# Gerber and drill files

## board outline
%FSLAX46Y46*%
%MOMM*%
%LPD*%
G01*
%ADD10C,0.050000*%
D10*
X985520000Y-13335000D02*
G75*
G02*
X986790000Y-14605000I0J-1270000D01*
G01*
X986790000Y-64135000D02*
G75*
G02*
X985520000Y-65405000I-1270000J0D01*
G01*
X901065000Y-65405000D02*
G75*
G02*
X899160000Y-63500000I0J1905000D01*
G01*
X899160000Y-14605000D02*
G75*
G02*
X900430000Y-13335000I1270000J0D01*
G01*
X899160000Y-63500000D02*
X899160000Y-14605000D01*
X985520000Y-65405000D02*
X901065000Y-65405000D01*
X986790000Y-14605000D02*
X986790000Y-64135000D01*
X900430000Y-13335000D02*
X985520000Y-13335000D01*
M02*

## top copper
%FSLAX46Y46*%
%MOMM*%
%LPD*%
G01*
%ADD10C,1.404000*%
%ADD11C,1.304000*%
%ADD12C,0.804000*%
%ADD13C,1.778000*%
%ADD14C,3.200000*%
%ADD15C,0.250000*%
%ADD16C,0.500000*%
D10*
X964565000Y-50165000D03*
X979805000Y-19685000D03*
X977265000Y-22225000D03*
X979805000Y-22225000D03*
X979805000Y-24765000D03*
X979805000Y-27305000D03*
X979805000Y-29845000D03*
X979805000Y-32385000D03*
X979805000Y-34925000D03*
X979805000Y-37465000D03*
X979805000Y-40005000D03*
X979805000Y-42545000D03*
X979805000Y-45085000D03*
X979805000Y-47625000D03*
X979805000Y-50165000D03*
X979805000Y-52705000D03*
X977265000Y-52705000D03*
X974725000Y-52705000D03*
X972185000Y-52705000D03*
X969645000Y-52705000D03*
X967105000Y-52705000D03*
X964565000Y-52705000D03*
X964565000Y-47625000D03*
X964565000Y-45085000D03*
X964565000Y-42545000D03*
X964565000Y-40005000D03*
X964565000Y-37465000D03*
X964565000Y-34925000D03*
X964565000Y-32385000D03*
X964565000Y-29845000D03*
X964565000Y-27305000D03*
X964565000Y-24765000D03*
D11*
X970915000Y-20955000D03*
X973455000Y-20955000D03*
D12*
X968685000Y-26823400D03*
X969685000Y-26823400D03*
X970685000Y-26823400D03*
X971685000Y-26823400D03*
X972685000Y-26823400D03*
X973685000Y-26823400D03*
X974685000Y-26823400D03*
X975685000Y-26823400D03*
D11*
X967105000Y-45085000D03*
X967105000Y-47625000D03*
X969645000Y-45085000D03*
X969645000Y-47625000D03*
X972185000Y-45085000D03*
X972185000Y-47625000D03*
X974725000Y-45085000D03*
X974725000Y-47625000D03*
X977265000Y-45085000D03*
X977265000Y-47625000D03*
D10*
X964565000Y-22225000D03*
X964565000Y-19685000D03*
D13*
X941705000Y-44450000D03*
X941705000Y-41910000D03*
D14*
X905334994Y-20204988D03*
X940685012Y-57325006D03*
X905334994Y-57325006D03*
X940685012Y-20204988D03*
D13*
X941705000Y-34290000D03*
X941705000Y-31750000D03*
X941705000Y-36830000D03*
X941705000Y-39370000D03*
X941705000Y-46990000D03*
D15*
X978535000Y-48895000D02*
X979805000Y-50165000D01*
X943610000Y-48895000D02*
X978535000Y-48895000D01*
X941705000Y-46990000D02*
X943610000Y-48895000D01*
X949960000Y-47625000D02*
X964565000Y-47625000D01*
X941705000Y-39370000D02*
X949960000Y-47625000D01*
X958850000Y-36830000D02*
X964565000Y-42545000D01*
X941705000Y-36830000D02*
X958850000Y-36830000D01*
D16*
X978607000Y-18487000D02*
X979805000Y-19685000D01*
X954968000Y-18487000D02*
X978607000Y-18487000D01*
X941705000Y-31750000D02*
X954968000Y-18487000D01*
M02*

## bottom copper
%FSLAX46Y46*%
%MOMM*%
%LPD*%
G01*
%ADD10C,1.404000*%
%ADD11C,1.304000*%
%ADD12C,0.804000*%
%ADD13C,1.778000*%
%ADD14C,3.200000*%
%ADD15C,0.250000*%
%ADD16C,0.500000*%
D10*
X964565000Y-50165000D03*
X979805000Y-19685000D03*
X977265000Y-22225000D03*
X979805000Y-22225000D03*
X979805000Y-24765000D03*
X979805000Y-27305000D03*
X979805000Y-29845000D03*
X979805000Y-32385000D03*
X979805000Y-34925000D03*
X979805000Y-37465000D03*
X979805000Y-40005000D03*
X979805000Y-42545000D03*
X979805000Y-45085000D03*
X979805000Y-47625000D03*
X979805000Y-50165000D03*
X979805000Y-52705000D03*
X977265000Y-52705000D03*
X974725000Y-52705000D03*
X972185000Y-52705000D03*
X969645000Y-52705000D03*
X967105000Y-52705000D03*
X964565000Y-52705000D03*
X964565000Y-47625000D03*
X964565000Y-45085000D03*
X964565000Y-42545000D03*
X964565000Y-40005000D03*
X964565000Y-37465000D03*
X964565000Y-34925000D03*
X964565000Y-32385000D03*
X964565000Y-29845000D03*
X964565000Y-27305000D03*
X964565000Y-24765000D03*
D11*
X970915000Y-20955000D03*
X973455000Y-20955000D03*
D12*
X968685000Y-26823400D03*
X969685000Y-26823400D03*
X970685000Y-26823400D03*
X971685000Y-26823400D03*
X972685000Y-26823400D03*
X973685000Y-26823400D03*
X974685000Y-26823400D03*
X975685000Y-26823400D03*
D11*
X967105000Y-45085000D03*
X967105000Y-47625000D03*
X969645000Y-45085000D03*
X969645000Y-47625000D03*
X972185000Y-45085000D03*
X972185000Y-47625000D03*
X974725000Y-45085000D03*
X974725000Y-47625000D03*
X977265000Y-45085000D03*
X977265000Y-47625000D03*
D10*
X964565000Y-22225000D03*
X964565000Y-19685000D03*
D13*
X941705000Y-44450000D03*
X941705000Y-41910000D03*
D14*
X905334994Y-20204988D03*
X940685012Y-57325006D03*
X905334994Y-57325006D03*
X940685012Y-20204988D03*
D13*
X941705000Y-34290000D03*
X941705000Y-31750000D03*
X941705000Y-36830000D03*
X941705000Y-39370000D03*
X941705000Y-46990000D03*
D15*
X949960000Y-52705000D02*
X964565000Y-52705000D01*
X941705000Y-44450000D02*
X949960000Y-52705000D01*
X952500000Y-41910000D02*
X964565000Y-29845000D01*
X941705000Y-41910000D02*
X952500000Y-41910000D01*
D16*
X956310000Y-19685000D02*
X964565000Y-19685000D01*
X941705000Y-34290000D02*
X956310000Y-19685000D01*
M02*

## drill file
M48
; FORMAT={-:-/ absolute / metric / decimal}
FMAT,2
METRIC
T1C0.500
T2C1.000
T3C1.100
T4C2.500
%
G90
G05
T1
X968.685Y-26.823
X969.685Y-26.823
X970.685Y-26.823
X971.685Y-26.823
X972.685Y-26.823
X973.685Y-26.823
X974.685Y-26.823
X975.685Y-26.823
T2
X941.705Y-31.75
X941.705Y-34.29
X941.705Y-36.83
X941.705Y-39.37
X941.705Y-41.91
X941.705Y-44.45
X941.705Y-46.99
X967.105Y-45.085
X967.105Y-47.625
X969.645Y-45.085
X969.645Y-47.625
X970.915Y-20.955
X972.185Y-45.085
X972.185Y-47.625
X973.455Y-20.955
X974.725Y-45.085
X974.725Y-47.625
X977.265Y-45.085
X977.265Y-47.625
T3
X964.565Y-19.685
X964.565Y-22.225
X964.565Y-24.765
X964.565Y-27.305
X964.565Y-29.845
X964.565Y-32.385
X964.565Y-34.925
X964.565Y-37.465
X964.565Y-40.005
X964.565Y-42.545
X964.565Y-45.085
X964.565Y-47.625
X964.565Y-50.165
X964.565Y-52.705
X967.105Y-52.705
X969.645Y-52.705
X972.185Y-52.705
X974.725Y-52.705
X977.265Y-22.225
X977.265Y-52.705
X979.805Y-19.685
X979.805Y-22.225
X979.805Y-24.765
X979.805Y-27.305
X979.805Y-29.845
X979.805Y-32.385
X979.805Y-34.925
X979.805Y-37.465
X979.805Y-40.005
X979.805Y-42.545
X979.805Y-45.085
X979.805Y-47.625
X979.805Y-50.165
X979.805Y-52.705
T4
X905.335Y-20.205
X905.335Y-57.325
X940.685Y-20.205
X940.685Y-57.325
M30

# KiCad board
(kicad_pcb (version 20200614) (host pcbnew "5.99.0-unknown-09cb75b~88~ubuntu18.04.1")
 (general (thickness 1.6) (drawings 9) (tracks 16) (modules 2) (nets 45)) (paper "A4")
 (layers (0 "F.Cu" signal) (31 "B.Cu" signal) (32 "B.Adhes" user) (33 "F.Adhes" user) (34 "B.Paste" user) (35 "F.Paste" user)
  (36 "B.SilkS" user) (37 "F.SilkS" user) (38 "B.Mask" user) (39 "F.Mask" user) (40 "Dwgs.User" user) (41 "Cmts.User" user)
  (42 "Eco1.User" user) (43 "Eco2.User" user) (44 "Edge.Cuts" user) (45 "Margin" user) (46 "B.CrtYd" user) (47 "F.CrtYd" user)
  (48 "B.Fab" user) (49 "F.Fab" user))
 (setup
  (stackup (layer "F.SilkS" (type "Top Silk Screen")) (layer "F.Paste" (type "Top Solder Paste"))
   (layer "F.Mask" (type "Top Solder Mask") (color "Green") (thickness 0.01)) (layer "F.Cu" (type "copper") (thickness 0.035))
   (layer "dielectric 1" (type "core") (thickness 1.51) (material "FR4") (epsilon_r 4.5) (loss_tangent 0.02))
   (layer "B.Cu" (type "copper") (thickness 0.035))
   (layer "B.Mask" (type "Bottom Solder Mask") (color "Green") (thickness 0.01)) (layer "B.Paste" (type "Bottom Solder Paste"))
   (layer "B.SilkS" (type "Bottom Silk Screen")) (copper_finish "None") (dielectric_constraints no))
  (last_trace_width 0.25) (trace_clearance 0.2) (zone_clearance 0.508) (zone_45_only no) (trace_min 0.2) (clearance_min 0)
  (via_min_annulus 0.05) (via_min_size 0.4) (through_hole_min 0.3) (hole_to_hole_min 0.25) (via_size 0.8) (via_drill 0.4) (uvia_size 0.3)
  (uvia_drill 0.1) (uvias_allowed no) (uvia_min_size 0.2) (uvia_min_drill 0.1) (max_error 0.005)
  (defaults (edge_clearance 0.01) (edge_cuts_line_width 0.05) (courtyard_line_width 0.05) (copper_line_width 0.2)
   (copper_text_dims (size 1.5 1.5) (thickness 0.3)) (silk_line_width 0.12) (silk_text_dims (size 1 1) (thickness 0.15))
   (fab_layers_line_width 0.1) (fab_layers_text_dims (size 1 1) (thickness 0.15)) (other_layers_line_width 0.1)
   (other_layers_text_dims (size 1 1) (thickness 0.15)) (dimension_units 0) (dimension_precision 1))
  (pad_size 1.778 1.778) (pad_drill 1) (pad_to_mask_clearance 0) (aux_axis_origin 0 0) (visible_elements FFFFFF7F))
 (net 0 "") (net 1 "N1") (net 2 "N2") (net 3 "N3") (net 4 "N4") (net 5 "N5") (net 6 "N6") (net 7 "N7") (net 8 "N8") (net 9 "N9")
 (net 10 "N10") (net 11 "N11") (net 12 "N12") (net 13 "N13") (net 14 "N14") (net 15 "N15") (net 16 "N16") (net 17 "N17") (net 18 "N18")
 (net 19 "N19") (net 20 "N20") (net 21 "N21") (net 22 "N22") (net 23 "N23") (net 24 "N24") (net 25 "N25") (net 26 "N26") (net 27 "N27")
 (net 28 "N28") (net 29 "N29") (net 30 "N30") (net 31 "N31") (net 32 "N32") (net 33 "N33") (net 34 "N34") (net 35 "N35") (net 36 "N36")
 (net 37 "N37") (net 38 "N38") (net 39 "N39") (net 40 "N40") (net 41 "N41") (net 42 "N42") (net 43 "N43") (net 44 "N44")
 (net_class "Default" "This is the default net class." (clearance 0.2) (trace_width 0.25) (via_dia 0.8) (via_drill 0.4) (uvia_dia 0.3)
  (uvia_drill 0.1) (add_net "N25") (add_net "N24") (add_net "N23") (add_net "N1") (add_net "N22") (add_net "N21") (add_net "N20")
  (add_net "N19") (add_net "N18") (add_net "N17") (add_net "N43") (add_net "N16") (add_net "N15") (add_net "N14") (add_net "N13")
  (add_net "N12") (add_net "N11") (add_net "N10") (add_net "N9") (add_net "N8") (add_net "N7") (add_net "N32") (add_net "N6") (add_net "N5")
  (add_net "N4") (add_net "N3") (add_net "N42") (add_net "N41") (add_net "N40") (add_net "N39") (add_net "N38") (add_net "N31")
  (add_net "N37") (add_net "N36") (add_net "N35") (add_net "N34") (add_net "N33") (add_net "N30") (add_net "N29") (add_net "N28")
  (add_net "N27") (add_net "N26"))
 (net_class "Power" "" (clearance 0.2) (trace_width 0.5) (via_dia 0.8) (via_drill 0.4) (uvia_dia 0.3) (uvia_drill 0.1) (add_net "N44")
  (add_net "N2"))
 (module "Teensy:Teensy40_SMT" (layer "F.Cu") (at 972.185 36.195 -90)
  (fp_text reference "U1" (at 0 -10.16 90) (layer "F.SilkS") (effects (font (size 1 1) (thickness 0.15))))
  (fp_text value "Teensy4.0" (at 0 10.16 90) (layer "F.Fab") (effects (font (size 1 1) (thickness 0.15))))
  (pad "13" thru_hole circle (at 13.97 7.62 270) (size 1.404 1.404) (drill 1.1) (layers *.Cu *.Mask) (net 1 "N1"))
  (pad "33" thru_hole circle (at -16.51 -7.62 270) (size 1.404 1.404) (drill 1.1) (layers *.Cu *.Mask) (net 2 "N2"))
  (pad "34" thru_hole circle (at -13.97 -5.08 270) (size 1.404 1.404) (drill 1.1) (layers *.Cu *.Mask) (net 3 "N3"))
  (pad "32" thru_hole circle (at -13.97 -7.62 270) (size 1.404 1.404) (drill 1.1) (layers *.Cu *.Mask) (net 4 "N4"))
  (pad "31" thru_hole circle (at -11.43 -7.62 270) (size 1.404 1.404) (drill 1.1) (layers *.Cu *.Mask) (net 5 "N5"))
  (pad "30" thru_hole circle (at -8.89 -7.62 270) (size 1.404 1.404) (drill 1.1) (layers *.Cu *.Mask) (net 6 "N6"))
  (pad "29" thru_hole circle (at -6.35 -7.62 270) (size 1.404 1.404) (drill 1.1) (layers *.Cu *.Mask) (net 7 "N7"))
  (pad "28" thru_hole circle (at -3.81 -7.62 270) (size 1.404 1.404) (drill 1.1) (layers *.Cu *.Mask) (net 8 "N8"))
  (pad "27" thru_hole circle (at -1.27 -7.62 270) (size 1.404 1.404) (drill 1.1) (layers *.Cu *.Mask) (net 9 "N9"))
  (pad "26" thru_hole circle (at 1.27 -7.62 270) (size 1.404 1.404) (drill 1.1) (layers *.Cu *.Mask) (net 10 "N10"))
  (pad "25" thru_hole circle (at 3.81 -7.62 270) (size 1.404 1.404) (drill 1.1) (layers *.Cu *.Mask) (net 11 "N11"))
  (pad "24" thru_hole circle (at 6.35 -7.62 270) (size 1.404 1.404) (drill 1.1) (layers *.Cu *.Mask) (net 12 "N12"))
  (pad "23" thru_hole circle (at 8.89 -7.62 270) (size 1.404 1.404) (drill 1.1) (layers *.Cu *.Mask) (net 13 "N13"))
  (pad "22" thru_hole circle (at 11.43 -7.62 270) (size 1.404 1.404) (drill 1.1) (layers *.Cu *.Mask) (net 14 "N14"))
  (pad "21" thru_hole circle (at 13.97 -7.62 270) (size 1.404 1.404) (drill 1.1) (layers *.Cu *.Mask) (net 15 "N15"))
  (pad "20" thru_hole circle (at 16.51 -7.62 270) (size 1.404 1.404) (drill 1.1) (layers *.Cu *.Mask) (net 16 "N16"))
  (pad "19" thru_hole circle (at 16.51 -5.08 270) (size 1.404 1.404) (drill 1.1) (layers *.Cu *.Mask) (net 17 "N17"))
  (pad "18" thru_hole circle (at 16.51 -2.54 270) (size 1.404 1.404) (drill 1.1) (layers *.Cu *.Mask) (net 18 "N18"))
  (pad "17" thru_hole circle (at 16.51 0 270) (size 1.404 1.404) (drill 1.1) (layers *.Cu *.Mask) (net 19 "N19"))
  (pad "16" thru_hole circle (at 16.51 2.54 270) (size 1.404 1.404) (drill 1.1) (layers *.Cu *.Mask) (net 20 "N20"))
  (pad "15" thru_hole circle (at 16.51 5.08 270) (size 1.404 1.404) (drill 1.1) (layers *.Cu *.Mask) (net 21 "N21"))
  (pad "14" thru_hole circle (at 16.51 7.62 270) (size 1.404 1.404) (drill 1.1) (layers *.Cu *.Mask) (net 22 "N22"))
  (pad "12" thru_hole circle (at 11.43 7.62 270) (size 1.404 1.404) (drill 1.1) (layers *.Cu *.Mask) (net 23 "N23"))
  (pad "11" thru_hole circle (at 8.89 7.62 270) (size 1.404 1.404) (drill 1.1) (layers *.Cu *.Mask) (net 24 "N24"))
  (pad "10" thru_hole circle (at 6.35 7.62 270) (size 1.404 1.404) (drill 1.1) (layers *.Cu *.Mask) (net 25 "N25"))
  (pad "9" thru_hole circle (at 3.81 7.62 270) (size 1.404 1.404) (drill 1.1) (layers *.Cu *.Mask) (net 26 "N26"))
  (pad "8" thru_hole circle (at 1.27 7.62 270) (size 1.404 1.404) (drill 1.1) (layers *.Cu *.Mask) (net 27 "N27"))
  (pad "7" thru_hole circle (at -1.27 7.62 270) (size 1.404 1.404) (drill 1.1) (layers *.Cu *.Mask) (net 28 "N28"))
  (pad "6" thru_hole circle (at -3.81 7.62 270) (size 1.404 1.404) (drill 1.1) (layers *.Cu *.Mask) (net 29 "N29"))
  (pad "5" thru_hole circle (at -6.35 7.62 270) (size 1.404 1.404) (drill 1.1) (layers *.Cu *.Mask) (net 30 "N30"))
  (pad "4" thru_hole circle (at -8.89 7.62 270) (size 1.404 1.404) (drill 1.1) (layers *.Cu *.Mask) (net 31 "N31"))
  (pad "3" thru_hole circle (at -11.43 7.62 270) (size 1.404 1.404) (drill 1.1) (layers *.Cu *.Mask) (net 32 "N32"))
  (pad "54" thru_hole circle (at -15.24 1.27 270) (size 1.304 1.304) (drill 1) (layers *.Cu *.Mask))
  (pad "53" thru_hole circle (at -15.24 -1.27 270) (size 1.304 1.304) (drill 1) (layers *.Cu *.Mask))
  (pad "52" thru_hole circle (at -9.3716 3.5 270) (size 0.804 0.804) (drill 0.5) (layers *.Cu *.Mask))
  (pad "51" thru_hole circle (at -9.3716 2.5 270) (size 0.804 0.804) (drill 0.5) (layers *.Cu *.Mask))
  (pad "50" thru_hole circle (at -9.3716 1.5 270) (size 0.804 0.804) (drill 0.5) (layers *.Cu *.Mask))
  (pad "49" thru_hole circle (at -9.3716 0.5 270) (size 0.804 0.804) (drill 0.5) (layers *.Cu *.Mask))
  (pad "48" thru_hole circle (at -9.3716 -0.5 270) (size 0.804 0.804) (drill 0.5) (layers *.Cu *.Mask))
  (pad "47" thru_hole circle (at -9.3716 -1.5 270) (size 0.804 0.804) (drill 0.5) (layers *.Cu *.Mask))
  (pad "46" thru_hole circle (at -9.3716 -2.5 270) (size 0.804 0.804) (drill 0.5) (layers *.Cu *.Mask))
  (pad "45" thru_hole circle (at -9.3716 -3.5 270) (size 0.804 0.804) (drill 0.5) (layers *.Cu *.Mask))
  (pad "44" thru_hole circle (at 8.89 5.08 270) (size 1.304 1.304) (drill 1) (layers *.Cu *.Mask) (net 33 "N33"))
  (pad "43" thru_hole circle (at 11.43 5.08 270) (size 1.304 1.304) (drill 1) (layers *.Cu *.Mask) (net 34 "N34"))
  (pad "42" thru_hole circle (at 8.89 2.54 270) (size 1.304 1.304) (drill 1) (layers *.Cu *.Mask) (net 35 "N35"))
  (pad "41" thru_hole circle (at 11.43 2.54 270) (size 1.304 1.304) (drill 1) (layers *.Cu *.Mask) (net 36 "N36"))
  (pad "40" thru_hole circle (at 8.89 0 270) (size 1.304 1.304) (drill 1) (layers *.Cu *.Mask) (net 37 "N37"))
  (pad "39" thru_hole circle (at 11.43 0 270) (size 1.304 1.304) (drill 1) (layers *.Cu *.Mask) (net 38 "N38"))
  (pad "38" thru_hole circle (at 8.89 -2.54 270) (size 1.304 1.304) (drill 1) (layers *.Cu *.Mask) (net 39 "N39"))
  (pad "37" thru_hole circle (at 11.43 -2.54 270) (size 1.304 1.304) (drill 1) (layers *.Cu *.Mask) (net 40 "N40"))
  (pad "36" thru_hole circle (at 8.89 -5.08 270) (size 1.304 1.304) (drill 1) (layers *.Cu *.Mask) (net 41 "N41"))
  (pad "35" thru_hole circle (at 11.43 -5.08 270) (size 1.304 1.304) (drill 1) (layers *.Cu *.Mask) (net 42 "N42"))
  (pad "2" thru_hole circle (at -13.97 7.62 270) (size 1.404 1.404) (drill 1.1) (layers *.Cu *.Mask) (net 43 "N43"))
  (pad "1" thru_hole circle (at -16.51 7.62 270) (size 1.404 1.404) (drill 1.1) (layers *.Cu *.Mask) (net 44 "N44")))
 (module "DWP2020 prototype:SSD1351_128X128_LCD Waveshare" (layer "F.Cu") (at 921.385 37.465)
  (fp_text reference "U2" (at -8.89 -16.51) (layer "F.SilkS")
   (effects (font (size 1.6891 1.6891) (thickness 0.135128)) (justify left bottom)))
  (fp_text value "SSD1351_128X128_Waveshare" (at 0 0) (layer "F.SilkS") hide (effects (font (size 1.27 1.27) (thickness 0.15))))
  (pad "JP1$6" thru_hole circle (at 20.32 6.985 90) (size 1.778 1.778) (drill 1) (layers *.Cu *.Mask) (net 22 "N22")
   (solder_mask_margin 0.1016))
  (pad "JP1$5" thru_hole circle (at 20.32 4.445 90) (size 1.778 1.778) (drill 1) (layers *.Cu *.Mask) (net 30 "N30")
   (solder_mask_margin 0.1016))
  (pad "U$26$P$1" thru_hole circle (at -16.050006 -17.260012) (size 3.2 3.2) (drill 2.5) (layers *.Cu *.Mask) (solder_mask_margin 0.1016))
  (pad "U$25$P$1" thru_hole circle (at 19.300012 19.860006) (size 3.2 3.2) (drill 2.5) (layers *.Cu *.Mask) (solder_mask_margin 0.1016))
  (pad "U$24$P$1" thru_hole circle (at -16.050006 19.860006) (size 3.2 3.2) (drill 2.5) (layers *.Cu *.Mask) (solder_mask_margin 0.1016))
  (pad "U$23$P$1" thru_hole circle (at 19.300012 -17.260012) (size 3.2 3.2) (drill 2.5) (layers *.Cu *.Mask) (solder_mask_margin 0.1016))
  (pad "JP1$2" thru_hole circle (at 20.32 -3.175 90) (size 1.778 1.778) (drill 1) (layers *.Cu *.Mask) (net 44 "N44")
   (solder_mask_margin 0.1016))
  (pad "JP1$1" thru_hole circle (at 20.32 -5.715 90) (size 1.778 1.778) (drill 1) (layers *.Cu *.Mask) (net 2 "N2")
   (solder_mask_margin 0.1016))
  (pad "JP1$3" thru_hole circle (at 20.32 -0.635 90) (size 1.778 1.778) (drill 1) (layers *.Cu *.Mask) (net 25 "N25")
   (solder_mask_margin 0.1016))
  (pad "JP1$4" thru_hole circle (at 20.32 1.905 90) (size 1.778 1.778) (drill 1) (layers *.Cu *.Mask) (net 23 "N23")
   (solder_mask_margin 0.1016))
  (pad "JP1$7" thru_hole circle (at 20.32 9.525 90) (size 1.778 1.778) (drill 1) (layers *.Cu *.Mask) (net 15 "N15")
   (solder_mask_margin 0.1016)))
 (gr_arc (start 985.52 14.605) (end 986.79 14.605) (angle -90) (layer "Edge.Cuts") (width 0.05))
 (gr_arc (start 985.52 64.135) (end 985.52 65.405) (angle -90) (layer "Edge.Cuts") (width 0.05))
 (gr_arc (start 901.065 63.5) (end 899.16 63.5) (angle -90) (layer "Edge.Cuts") (width 0.05))
 (gr_arc (start 900.43 14.605) (end 900.43 13.335) (angle -90) (layer "Edge.Cuts") (width 0.05))
 (gr_line (start 899.16 63.5) (end 899.16 14.605) (layer "Edge.Cuts") (width 0.05))
 (gr_line (start 985.52 65.405) (end 901.065 65.405) (layer "Edge.Cuts") (width 0.05))
 (gr_line (start 986.79 14.605) (end 986.79 64.135) (layer "Edge.Cuts") (width 0.05))
 (gr_line (start 900.43 13.335) (end 985.52 13.335) (layer "Edge.Cuts") (width 0.05))
 (segment (start 949.96 52.705) (end 964.565 52.705) (width 0.25) (layer "B.Cu") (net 22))
 (segment (start 941.705 44.45) (end 949.96 52.705) (width 0.25) (layer "B.Cu") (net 22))
 (segment (start 978.535 48.895) (end 979.805 50.165) (width 0.25) (layer "F.Cu") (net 15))
 (segment (start 943.61 48.895) (end 978.535 48.895) (width 0.25) (layer "F.Cu") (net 15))
 (segment (start 941.705 46.99) (end 943.61 48.895) (width 0.25) (layer "F.Cu") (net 15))
 (segment (start 949.96 47.625) (end 964.565 47.625) (width 0.25) (layer "F.Cu") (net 23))
 (segment (start 941.705 39.37) (end 949.96 47.625) (width 0.25) (layer "F.Cu") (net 23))
 (segment (start 958.85 36.83) (end 964.565 42.545) (width 0.25) (layer "F.Cu") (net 25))
 (segment (start 941.705 36.83) (end 958.85 36.83) (width 0.25) (layer "F.Cu") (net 25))
 (segment (start 952.5 41.91) (end 964.565 29.845) (width 0.25) (layer "B.Cu") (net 30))
 (segment (start 941.705 41.91) (end 952.5 41.91) (width 0.25) (layer "B.Cu") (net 30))
 (segment (start 956.31 19.685) (end 964.565 19.685) (width 0.5) (layer "B.Cu") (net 44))
 (segment (start 941.705 34.29) (end 956.31 19.685) (width 0.5) (layer "B.Cu") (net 44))
 (segment (start 978.607 18.487) (end 979.805 19.685) (width 0.5) (layer "F.Cu") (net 2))
 (segment (start 954.968 18.487) (end 978.607 18.487) (width 0.5) (layer "F.Cu") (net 2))
 (segment (start 941.705 31.75) (end 954.968 18.487) (width 0.5) (layer "F.Cu") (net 2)))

